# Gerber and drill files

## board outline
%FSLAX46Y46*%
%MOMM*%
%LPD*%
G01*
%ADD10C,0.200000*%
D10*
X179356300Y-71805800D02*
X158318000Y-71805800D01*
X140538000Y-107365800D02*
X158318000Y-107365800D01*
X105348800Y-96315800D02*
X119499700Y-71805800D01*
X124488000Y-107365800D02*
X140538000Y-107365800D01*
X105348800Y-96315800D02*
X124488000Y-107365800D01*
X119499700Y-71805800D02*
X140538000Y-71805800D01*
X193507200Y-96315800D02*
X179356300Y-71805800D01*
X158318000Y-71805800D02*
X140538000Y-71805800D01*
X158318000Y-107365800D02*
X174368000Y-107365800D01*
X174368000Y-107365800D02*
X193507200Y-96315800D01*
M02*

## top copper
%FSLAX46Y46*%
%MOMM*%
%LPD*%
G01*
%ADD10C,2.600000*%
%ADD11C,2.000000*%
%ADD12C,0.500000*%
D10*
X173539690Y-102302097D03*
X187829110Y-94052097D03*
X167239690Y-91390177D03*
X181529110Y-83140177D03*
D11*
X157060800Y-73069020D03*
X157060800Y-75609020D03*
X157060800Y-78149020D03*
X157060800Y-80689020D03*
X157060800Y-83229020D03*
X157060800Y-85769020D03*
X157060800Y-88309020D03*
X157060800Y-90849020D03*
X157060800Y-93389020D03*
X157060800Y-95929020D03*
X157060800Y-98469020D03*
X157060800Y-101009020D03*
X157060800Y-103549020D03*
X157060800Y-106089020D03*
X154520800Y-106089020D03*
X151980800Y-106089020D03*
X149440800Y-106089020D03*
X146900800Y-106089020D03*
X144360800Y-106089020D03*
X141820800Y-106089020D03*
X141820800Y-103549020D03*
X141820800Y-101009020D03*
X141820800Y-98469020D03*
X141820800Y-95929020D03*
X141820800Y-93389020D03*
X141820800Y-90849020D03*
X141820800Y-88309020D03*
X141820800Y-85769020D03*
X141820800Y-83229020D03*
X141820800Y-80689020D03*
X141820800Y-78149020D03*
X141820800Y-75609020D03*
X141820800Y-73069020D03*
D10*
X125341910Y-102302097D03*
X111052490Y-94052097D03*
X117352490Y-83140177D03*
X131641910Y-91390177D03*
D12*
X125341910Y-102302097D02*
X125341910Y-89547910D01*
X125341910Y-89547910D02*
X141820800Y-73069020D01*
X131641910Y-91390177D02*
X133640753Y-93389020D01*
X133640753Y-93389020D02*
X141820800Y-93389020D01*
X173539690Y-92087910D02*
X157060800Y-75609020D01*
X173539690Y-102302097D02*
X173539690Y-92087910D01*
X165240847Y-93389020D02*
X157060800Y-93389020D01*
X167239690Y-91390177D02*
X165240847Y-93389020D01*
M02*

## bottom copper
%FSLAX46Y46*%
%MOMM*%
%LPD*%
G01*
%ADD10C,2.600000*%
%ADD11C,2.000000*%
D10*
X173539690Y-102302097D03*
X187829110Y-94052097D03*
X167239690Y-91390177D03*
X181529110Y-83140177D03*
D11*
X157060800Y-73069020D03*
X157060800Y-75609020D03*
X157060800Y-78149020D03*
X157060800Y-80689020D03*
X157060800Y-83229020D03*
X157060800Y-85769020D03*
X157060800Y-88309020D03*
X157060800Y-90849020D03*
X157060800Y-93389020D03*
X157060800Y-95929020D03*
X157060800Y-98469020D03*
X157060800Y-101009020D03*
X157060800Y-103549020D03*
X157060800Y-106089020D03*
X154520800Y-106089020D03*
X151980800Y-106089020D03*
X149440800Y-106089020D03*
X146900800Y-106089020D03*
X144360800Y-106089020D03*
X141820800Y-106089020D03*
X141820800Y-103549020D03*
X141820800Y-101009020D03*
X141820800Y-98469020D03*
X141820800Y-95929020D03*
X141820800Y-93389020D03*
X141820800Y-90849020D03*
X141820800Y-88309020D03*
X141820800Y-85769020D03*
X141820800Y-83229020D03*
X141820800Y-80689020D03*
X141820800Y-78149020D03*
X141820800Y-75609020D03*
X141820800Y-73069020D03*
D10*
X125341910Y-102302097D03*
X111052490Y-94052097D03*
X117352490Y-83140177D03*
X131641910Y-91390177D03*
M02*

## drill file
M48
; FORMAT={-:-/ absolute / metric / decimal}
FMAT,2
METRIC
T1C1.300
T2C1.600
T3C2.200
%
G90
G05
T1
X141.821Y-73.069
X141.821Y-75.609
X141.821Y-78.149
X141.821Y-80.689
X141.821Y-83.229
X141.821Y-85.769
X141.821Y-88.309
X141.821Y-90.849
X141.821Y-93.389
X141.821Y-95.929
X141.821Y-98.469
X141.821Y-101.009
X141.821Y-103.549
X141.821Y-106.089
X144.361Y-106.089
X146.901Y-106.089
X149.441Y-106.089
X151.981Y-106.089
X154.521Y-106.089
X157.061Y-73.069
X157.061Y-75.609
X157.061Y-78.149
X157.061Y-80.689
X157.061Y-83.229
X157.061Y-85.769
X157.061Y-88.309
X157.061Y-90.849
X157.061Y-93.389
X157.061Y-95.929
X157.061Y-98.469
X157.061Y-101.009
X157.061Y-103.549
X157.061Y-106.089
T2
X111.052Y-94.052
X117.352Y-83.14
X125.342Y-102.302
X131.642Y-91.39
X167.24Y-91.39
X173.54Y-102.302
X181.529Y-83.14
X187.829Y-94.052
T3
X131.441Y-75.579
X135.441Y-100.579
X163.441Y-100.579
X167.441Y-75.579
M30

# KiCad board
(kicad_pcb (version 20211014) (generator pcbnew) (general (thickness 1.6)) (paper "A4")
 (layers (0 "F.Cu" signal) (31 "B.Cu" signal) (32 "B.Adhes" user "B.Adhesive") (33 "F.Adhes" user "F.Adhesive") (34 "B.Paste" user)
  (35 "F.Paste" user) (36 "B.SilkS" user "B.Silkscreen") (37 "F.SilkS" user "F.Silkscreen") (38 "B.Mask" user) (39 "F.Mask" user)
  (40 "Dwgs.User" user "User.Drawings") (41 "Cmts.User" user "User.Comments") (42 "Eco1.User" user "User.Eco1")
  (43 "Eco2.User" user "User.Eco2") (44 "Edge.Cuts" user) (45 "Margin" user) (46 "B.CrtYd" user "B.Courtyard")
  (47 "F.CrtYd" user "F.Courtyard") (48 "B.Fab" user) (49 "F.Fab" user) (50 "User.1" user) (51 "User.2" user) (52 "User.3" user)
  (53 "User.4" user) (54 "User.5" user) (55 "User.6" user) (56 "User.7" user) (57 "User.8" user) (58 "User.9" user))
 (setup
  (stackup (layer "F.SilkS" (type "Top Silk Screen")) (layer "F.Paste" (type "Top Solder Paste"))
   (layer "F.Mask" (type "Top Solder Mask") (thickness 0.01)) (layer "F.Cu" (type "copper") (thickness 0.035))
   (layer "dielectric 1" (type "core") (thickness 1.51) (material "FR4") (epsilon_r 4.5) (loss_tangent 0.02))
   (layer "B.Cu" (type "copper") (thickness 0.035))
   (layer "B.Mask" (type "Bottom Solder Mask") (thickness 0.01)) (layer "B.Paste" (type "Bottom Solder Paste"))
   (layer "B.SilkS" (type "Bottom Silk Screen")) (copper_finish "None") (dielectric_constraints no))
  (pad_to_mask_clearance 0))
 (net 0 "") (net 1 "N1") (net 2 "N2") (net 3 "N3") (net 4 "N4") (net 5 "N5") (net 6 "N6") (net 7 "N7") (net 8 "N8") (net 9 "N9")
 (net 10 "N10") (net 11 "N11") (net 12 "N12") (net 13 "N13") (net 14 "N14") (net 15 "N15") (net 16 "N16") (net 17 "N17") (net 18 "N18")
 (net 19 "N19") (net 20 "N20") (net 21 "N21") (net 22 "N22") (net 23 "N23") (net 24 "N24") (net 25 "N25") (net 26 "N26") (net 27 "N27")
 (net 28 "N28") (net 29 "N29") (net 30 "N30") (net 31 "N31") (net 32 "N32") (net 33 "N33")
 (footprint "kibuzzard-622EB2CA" (layer "F.Cu") (at 149.4028 74.1934)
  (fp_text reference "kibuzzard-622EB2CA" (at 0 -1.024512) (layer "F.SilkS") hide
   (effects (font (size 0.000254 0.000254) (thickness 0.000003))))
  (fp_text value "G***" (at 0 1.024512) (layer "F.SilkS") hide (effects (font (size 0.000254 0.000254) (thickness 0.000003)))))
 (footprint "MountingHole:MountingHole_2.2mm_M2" (layer "F.Cu") (at 135.4408 100.57902)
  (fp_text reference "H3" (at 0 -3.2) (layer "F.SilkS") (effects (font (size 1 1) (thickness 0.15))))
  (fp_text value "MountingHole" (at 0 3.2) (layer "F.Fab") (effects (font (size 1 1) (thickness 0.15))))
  (pad "" np_thru_hole circle (at 0 0) (size 2.2 2.2) (drill 2.2) (layers *.Cu *.Mask)))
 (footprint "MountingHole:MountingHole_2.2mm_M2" (layer "F.Cu") (at 131.4408 75.57902)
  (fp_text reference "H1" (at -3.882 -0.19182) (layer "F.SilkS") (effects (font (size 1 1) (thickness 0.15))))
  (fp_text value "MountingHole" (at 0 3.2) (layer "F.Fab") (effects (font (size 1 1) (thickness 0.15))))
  (pad "" np_thru_hole circle (at 0 0) (size 2.2 2.2) (drill 2.2) (layers *.Cu *.Mask)))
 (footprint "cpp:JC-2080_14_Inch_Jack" (layer "F.Cu") (at 176.8094 91.4654 -150)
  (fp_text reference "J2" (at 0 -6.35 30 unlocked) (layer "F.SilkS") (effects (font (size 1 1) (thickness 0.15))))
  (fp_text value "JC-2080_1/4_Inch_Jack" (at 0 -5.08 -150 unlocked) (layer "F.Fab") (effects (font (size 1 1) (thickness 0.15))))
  (pad "1" thru_hole circle (at 8.25 -7.75 210) (size 2.6 2.6) (drill 1.6) (layers *.Cu *.Mask) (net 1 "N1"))
  (pad "1" thru_hole circle (at -8.25 -7.75 210) (size 2.6 2.6) (drill 1.6) (layers *.Cu *.Mask) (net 1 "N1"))
  (pad "2" thru_hole circle (at 8.25 4.85 210) (size 2.6 2.6) (drill 1.6) (layers *.Cu *.Mask) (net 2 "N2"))
  (pad "2" thru_hole circle (at -8.25 4.85 210) (size 2.6 2.6) (drill 1.6) (layers *.Cu *.Mask) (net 2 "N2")))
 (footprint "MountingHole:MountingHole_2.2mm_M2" (layer "F.Cu") (at 167.4408 75.57902)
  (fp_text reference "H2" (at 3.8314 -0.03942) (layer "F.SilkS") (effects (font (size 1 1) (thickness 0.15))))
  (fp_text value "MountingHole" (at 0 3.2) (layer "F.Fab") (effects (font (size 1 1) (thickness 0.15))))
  (pad "" np_thru_hole circle (at 0 0) (size 2.2 2.2) (drill 2.2) (layers *.Cu *.Mask)))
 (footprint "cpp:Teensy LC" (layer "F.Cu") (at 149.4408 89.57902)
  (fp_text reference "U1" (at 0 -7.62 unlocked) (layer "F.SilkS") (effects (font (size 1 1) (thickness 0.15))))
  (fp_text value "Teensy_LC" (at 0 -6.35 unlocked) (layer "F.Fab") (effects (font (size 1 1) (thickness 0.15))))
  (pad "1" thru_hole circle (at 7.62 -16.51) (size 2 2) (drill 1.3) (layers *.Cu *.Mask) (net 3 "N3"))
  (pad "2" thru_hole circle (at 7.62 -13.97) (size 2 2) (drill 1.3) (layers *.Cu *.Mask) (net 1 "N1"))
  (pad "3" thru_hole circle (at 7.62 -11.43) (size 2 2) (drill 1.3) (layers *.Cu *.Mask) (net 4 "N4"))
  (pad "4" thru_hole circle (at 7.62 -8.89) (size 2 2) (drill 1.3) (layers *.Cu *.Mask) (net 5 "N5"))
  (pad "5" thru_hole circle (at 7.62 -6.35) (size 2 2) (drill 1.3) (layers *.Cu *.Mask) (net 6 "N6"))
  (pad "6" thru_hole circle (at 7.62 -3.81) (size 2 2) (drill 1.3) (layers *.Cu *.Mask) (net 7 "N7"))
  (pad "7" thru_hole circle (at 7.62 -1.27) (size 2 2) (drill 1.3) (layers *.Cu *.Mask) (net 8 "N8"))
  (pad "8" thru_hole circle (at 7.62 1.27) (size 2 2) (drill 1.3) (layers *.Cu *.Mask) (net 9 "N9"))
  (pad "9" thru_hole circle (at 7.62 3.81) (size 2 2) (drill 1.3) (layers *.Cu *.Mask) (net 2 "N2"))
  (pad "10" thru_hole circle (at 7.62 6.35) (size 2 2) (drill 1.3) (layers *.Cu *.Mask) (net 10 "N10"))
  (pad "11" thru_hole circle (at 7.62 8.89) (size 2 2) (drill 1.3) (layers *.Cu *.Mask) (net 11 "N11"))
  (pad "12" thru_hole circle (at 7.62 11.43) (size 2 2) (drill 1.3) (layers *.Cu *.Mask) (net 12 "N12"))
  (pad "13" thru_hole circle (at 7.62 13.97) (size 2 2) (drill 1.3) (layers *.Cu *.Mask) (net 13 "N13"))
  (pad "14" thru_hole circle (at 7.62 16.51) (size 2 2) (drill 1.3) (layers *.Cu *.Mask) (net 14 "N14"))
  (pad "15" thru_hole circle (at 5.08 16.51) (size 2 2) (drill 1.3) (layers *.Cu *.Mask) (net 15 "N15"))
  (pad "16" thru_hole circle (at 2.54 16.51) (size 2 2) (drill 1.3) (layers *.Cu *.Mask) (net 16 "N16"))
  (pad "17" thru_hole circle (at 0 16.51) (size 2 2) (drill 1.3) (layers *.Cu *.Mask) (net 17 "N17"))
  (pad "18" thru_hole circle (at -2.54 16.51) (size 2 2) (drill 1.3) (layers *.Cu *.Mask) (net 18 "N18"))
  (pad "19" thru_hole circle (at -5.08 16.51) (size 2 2) (drill 1.3) (layers *.Cu *.Mask) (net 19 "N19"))
  (pad "20" thru_hole circle (at -7.62 16.51) (size 2 2) (drill 1.3) (layers *.Cu *.Mask) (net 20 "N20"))
  (pad "21" thru_hole circle (at -7.62 13.97) (size 2 2) (drill 1.3) (layers *.Cu *.Mask) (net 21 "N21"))
  (pad "22" thru_hole circle (at -7.62 11.43) (size 2 2) (drill 1.3) (layers *.Cu *.Mask) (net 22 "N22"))
  (pad "23" thru_hole circle (at -7.62 8.89) (size 2 2) (drill 1.3) (layers *.Cu *.Mask) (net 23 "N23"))
  (pad "24" thru_hole circle (at -7.62 6.35) (size 2 2) (drill 1.3) (layers *.Cu *.Mask) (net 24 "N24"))
  (pad "25" thru_hole circle (at -7.62 3.81) (size 2 2) (drill 1.3) (layers *.Cu *.Mask) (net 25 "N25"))
  (pad "26" thru_hole circle (at -7.62 1.27) (size 2 2) (drill 1.3) (layers *.Cu *.Mask) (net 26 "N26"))
  (pad "27" thru_hole circle (at -7.62 -1.27) (size 2 2) (drill 1.3) (layers *.Cu *.Mask) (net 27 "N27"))
  (pad "28" thru_hole circle (at -7.62 -3.81) (size 2 2) (drill 1.3) (layers *.Cu *.Mask) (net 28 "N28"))
  (pad "29" thru_hole circle (at -7.62 -6.35) (size 2 2) (drill 1.3) (layers *.Cu *.Mask) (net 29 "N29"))
  (pad "30" thru_hole circle (at -7.62 -8.89) (size 2 2) (drill 1.3) (layers *.Cu *.Mask) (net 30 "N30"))
  (pad "31" thru_hole circle (at -7.62 -11.43) (size 2 2) (drill 1.3) (layers *.Cu *.Mask) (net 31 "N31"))
  (pad "32" thru_hole circle (at -7.62 -13.97) (size 2 2) (drill 1.3) (layers *.Cu *.Mask) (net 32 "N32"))
  (pad "33" thru_hole circle (at -7.62 -16.51) (size 2 2) (drill 1.3) (layers *.Cu *.Mask) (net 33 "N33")))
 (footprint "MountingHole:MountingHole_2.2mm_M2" (layer "F.Cu") (at 163.4408 100.57902)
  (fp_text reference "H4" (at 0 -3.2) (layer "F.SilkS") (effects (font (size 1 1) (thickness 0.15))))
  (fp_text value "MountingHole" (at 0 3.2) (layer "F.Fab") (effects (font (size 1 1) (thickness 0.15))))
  (pad "" np_thru_hole circle (at 0 0) (size 2.2 2.2) (drill 2.2) (layers *.Cu *.Mask)))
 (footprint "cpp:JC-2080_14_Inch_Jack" (layer "F.Cu") (at 122.0722 91.4654 150)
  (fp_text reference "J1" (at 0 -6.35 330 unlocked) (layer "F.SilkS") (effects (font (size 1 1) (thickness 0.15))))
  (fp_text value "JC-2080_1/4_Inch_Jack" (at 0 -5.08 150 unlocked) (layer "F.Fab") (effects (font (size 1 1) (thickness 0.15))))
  (pad "1" thru_hole circle (at -8.25 -7.75 150) (size 2.6 2.6) (drill 1.6) (layers *.Cu *.Mask) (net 33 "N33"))
  (pad "1" thru_hole circle (at 8.25 -7.75 150) (size 2.6 2.6) (drill 1.6) (layers *.Cu *.Mask) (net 33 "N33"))
  (pad "2" thru_hole circle (at 8.25 4.85 150) (size 2.6 2.6) (drill 1.6) (layers *.Cu *.Mask) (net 25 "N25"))
  (pad "2" thru_hole circle (at -8.25 4.85 150) (size 2.6 2.6) (drill 1.6) (layers *.Cu *.Mask) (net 25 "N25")))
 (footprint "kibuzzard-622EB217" (layer "B.Cu") (at 121.9962 92.0242 150)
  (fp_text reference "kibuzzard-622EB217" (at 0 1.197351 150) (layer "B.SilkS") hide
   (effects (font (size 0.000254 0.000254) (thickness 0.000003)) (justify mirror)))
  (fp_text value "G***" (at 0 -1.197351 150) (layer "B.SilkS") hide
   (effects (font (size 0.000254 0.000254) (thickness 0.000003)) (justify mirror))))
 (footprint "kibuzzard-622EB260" (layer "B.Cu") (at 120.0658 94.8944 150)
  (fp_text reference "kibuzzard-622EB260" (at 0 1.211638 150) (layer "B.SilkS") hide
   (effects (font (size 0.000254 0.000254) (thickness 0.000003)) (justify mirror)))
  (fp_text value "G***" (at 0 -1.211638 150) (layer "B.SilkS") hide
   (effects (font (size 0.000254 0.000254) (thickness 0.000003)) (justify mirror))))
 (gr_line (start 179.3563 71.8058) (end 158.318 71.8058) (layer "Edge.Cuts") (width 0.2))
 (gr_line (start 140.538 107.3658) (end 158.318 107.3658) (layer "Edge.Cuts") (width 0.2))
 (gr_line (start 105.3488 96.3158) (end 119.4997 71.8058) (layer "Edge.Cuts") (width 0.2))
 (gr_line (start 124.488 107.3658) (end 140.538 107.3658) (layer "Edge.Cuts") (width 0.2))
 (gr_line (start 105.3488 96.3158) (end 124.488 107.3658) (layer "Edge.Cuts") (width 0.2))
 (gr_line (start 119.4997 71.8058) (end 140.538 71.8058) (layer "Edge.Cuts") (width 0.2))
 (gr_line (start 193.5072 96.3158) (end 179.3563 71.8058) (layer "Edge.Cuts") (width 0.2))
 (gr_line (start 158.318 71.8058) (end 140.538 71.8058) (layer "Edge.Cuts") (width 0.2))
 (gr_line (start 158.318 107.3658) (end 174.368 107.3658) (layer "Edge.Cuts") (width 0.2))
 (gr_line (start 174.368 107.3658) (end 193.5072 96.3158) (layer "Edge.Cuts") (width 0.2))
 (segment (start 125.34191 102.302097) (end 125.34191 89.54791) (width 0.5) (layer "F.Cu") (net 33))
 (segment (start 125.34191 89.54791) (end 141.8208 73.06902) (width 0.5) (layer "F.Cu") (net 33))
 (segment (start 131.64191 91.390177) (end 133.640753 93.38902) (width 0.5) (layer "F.Cu") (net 25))
 (segment (start 133.640753 93.38902) (end 141.8208 93.38902) (width 0.5) (layer "F.Cu") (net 25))
 (segment (start 173.53969 92.08791) (end 157.0608 75.60902) (width 0.5) (layer "F.Cu") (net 1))
 (segment (start 173.53969 102.302097) (end 173.53969 92.08791) (width 0.5) (layer "F.Cu") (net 1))
 (segment (start 165.240847 93.38902) (end 157.0608 93.38902) (width 0.5) (layer "F.Cu") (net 2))
 (segment (start 167.23969 91.390177) (end 165.240847 93.38902) (width 0.5) (layer "F.Cu") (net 2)))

